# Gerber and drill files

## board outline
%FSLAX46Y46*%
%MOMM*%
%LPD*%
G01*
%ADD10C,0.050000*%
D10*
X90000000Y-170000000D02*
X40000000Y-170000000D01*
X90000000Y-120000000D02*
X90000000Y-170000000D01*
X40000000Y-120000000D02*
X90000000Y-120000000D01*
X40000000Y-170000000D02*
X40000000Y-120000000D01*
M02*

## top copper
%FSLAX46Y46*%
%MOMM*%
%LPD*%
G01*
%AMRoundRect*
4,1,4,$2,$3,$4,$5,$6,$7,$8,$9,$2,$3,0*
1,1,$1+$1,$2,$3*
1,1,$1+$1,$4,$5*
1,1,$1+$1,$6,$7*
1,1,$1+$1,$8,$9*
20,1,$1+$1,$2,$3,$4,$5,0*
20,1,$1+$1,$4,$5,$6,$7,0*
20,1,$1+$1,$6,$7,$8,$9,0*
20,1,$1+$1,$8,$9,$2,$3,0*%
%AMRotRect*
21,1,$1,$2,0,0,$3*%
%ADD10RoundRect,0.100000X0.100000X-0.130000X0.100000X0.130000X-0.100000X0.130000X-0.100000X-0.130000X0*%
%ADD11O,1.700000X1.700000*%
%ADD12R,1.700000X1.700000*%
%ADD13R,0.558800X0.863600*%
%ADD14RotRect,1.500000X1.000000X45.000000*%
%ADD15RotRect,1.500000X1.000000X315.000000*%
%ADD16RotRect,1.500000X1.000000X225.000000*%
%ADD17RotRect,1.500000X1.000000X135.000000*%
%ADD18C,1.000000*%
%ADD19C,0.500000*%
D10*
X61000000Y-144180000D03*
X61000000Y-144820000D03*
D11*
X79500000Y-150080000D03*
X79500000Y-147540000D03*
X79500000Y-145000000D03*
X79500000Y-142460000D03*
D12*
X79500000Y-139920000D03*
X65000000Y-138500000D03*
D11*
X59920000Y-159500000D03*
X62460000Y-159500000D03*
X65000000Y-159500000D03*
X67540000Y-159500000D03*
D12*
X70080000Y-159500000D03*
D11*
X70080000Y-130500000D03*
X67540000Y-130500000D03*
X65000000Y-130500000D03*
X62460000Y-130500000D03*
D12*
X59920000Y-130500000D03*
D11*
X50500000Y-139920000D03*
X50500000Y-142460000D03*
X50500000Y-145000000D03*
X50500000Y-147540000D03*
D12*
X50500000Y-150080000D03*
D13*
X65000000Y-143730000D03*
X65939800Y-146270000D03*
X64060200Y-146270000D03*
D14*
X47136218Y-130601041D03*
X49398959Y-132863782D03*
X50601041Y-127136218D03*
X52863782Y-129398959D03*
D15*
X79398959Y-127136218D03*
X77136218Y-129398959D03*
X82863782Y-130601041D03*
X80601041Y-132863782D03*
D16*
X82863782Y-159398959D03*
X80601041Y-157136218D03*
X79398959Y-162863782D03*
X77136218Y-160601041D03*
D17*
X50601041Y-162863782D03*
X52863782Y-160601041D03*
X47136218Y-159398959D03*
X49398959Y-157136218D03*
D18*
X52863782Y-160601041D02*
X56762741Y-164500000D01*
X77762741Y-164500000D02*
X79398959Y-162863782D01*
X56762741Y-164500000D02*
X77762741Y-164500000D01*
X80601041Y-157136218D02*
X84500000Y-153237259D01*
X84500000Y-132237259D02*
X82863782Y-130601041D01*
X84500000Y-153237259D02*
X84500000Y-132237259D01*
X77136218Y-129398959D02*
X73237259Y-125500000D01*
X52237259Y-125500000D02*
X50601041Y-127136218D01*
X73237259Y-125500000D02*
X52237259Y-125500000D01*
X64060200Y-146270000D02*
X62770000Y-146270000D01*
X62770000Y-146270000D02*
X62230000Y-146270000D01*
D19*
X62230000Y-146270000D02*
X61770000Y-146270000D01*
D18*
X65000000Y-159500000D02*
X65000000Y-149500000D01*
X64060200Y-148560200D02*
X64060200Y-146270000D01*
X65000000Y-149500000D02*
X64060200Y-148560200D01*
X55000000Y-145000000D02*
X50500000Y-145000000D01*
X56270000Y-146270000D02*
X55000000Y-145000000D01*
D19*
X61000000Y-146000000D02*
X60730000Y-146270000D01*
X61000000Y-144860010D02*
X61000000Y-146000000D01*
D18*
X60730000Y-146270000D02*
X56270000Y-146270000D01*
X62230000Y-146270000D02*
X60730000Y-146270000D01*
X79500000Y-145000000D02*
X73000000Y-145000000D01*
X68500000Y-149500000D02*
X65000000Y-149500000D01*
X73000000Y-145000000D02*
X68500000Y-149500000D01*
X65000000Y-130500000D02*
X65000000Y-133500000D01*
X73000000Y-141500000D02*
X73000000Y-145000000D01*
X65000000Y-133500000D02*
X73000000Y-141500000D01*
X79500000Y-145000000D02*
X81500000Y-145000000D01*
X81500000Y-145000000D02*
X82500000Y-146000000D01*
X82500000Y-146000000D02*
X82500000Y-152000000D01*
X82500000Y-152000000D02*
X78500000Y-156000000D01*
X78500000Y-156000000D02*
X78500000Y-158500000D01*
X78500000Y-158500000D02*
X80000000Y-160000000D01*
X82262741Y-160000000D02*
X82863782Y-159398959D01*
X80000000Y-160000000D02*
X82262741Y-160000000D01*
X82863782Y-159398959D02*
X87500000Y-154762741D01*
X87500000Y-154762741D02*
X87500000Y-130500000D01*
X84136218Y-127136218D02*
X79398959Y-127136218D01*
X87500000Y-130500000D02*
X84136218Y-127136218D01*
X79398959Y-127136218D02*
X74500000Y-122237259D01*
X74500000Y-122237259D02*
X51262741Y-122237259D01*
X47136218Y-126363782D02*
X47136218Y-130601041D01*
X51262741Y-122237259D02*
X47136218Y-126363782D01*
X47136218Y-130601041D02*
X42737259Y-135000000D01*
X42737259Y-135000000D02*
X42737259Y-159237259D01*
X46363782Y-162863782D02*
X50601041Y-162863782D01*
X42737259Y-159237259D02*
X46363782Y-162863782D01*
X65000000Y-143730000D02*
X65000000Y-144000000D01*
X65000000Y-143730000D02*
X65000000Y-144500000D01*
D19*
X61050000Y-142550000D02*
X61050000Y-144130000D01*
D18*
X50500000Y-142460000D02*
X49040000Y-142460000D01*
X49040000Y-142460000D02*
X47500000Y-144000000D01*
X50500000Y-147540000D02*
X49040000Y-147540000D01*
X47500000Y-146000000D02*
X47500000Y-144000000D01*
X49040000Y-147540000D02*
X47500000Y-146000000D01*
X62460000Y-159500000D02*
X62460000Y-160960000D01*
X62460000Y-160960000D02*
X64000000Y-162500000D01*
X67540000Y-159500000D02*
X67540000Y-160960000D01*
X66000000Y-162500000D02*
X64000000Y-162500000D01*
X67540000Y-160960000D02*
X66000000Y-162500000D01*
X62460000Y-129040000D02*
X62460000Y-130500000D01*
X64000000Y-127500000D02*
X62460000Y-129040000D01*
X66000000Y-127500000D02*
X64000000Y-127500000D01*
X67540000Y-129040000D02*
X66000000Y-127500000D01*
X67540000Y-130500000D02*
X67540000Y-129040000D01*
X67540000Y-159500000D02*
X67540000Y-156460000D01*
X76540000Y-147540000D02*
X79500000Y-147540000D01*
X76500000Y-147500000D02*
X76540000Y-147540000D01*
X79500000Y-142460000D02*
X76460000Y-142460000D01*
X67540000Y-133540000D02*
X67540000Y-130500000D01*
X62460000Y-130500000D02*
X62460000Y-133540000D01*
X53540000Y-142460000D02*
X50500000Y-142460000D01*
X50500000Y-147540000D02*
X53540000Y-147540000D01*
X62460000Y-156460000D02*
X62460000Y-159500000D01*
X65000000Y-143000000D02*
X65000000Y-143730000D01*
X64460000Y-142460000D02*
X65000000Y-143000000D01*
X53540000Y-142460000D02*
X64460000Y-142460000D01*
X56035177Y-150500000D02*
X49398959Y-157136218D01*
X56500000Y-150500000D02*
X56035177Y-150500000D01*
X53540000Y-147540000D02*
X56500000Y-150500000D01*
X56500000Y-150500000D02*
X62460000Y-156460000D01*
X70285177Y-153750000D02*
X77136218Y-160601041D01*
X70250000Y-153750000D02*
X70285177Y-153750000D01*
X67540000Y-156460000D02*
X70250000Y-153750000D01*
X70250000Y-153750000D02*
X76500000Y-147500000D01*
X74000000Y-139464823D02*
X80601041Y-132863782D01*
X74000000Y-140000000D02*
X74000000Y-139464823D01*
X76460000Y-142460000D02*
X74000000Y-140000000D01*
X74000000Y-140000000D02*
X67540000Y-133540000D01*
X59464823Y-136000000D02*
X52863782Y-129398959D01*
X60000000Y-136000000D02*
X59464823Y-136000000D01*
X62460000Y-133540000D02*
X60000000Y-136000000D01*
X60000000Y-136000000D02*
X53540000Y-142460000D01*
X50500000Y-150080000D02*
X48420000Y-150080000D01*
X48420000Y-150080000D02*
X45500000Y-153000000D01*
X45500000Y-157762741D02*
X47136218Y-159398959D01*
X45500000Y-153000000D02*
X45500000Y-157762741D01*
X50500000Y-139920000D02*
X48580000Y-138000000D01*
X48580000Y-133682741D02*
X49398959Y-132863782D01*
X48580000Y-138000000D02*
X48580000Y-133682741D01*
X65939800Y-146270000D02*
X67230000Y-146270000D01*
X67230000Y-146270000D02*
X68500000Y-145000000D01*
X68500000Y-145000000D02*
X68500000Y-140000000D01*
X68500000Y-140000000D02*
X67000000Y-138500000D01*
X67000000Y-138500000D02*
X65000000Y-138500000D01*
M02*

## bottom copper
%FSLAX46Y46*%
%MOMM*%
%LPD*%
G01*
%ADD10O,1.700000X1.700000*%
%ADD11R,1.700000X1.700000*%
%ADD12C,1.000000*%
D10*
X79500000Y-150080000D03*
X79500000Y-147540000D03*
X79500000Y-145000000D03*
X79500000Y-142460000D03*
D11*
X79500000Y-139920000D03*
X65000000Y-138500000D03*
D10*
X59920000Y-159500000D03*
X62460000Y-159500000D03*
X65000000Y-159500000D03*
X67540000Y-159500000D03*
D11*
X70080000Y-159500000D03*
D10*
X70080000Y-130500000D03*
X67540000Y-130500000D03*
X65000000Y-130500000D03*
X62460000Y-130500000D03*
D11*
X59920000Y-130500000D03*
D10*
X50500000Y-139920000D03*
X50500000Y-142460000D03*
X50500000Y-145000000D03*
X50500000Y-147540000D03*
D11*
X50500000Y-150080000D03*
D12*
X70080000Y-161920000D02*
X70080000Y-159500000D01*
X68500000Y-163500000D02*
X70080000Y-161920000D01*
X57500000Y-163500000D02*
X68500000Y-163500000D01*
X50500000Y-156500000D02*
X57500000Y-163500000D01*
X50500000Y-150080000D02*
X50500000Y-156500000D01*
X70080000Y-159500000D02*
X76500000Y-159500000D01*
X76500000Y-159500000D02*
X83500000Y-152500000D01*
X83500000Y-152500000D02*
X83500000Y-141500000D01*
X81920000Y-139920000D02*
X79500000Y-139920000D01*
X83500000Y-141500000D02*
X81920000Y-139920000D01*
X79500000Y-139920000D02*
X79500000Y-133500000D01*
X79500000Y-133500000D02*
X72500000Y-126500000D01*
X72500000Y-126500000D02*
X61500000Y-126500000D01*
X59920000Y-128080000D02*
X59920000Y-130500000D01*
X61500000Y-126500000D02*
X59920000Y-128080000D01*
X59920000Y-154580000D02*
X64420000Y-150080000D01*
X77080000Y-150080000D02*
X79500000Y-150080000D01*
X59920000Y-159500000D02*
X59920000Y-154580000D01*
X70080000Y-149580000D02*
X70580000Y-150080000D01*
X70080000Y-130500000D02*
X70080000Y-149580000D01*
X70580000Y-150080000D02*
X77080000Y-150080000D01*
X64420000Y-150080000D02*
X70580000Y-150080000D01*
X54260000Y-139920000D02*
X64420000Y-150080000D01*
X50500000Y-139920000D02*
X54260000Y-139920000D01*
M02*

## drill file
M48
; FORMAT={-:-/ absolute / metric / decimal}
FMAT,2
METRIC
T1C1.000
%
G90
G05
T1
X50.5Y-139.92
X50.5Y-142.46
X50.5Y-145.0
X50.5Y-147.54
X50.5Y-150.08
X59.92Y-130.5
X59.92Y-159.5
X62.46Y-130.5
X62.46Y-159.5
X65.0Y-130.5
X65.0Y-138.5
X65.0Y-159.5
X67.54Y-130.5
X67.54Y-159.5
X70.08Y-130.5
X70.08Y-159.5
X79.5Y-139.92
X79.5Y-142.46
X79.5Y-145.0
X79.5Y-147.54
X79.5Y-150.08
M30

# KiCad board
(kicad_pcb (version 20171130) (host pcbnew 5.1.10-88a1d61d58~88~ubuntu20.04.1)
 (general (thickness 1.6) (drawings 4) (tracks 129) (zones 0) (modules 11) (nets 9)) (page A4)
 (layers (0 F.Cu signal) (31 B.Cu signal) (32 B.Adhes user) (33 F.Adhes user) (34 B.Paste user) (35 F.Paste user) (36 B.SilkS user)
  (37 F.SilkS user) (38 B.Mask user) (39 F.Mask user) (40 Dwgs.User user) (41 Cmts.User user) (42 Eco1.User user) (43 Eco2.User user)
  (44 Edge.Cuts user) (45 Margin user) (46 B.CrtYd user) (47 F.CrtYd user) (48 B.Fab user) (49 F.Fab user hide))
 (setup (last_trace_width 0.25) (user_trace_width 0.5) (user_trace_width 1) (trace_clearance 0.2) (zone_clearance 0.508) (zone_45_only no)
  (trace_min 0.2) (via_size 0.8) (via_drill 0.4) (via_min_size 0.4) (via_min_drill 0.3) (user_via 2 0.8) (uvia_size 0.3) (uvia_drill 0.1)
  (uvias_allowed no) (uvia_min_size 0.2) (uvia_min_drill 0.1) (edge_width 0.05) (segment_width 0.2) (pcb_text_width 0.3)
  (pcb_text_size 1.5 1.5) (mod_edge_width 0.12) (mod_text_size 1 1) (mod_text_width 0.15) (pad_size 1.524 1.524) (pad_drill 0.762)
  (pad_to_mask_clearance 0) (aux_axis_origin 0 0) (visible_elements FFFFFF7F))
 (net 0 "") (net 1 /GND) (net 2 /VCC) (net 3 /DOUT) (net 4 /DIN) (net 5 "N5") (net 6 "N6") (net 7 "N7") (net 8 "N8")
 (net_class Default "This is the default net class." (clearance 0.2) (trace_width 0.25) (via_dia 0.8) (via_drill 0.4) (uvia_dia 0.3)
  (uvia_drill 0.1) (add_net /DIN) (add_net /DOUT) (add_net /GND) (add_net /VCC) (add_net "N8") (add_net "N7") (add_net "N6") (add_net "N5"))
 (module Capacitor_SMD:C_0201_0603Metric (layer F.Cu) (at 61 144.5 90)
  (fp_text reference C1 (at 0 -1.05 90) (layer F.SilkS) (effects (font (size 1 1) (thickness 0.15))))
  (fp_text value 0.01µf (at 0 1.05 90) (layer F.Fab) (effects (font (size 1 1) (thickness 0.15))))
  (pad 2 smd roundrect (at 0.32 0 90) (size 0.46 0.4) (layers F.Cu F.Mask) (roundrect_rratio 0.25) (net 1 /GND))
  (pad 1 smd roundrect (at -0.32 0 90) (size 0.46 0.4) (layers F.Cu F.Mask) (roundrect_rratio 0.25) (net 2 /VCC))
  (pad "" smd roundrect (at 0.345 0 90) (size 0.318 0.36) (layers F.Paste) (roundrect_rratio 0.25))
  (pad "" smd roundrect (at -0.345 0 90) (size 0.318 0.36) (layers F.Paste) (roundrect_rratio 0.25)))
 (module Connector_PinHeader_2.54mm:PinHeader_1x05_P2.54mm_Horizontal (layer F.Cu) (at 79.5 139.92)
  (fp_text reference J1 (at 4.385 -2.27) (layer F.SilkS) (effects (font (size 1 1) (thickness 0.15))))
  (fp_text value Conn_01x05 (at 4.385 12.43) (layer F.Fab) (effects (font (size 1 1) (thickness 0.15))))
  (pad 5 thru_hole oval (at 0 10.16) (size 1.7 1.7) (drill 1) (layers *.Cu *.Mask) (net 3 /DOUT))
  (pad 4 thru_hole oval (at 0 7.62) (size 1.7 1.7) (drill 1) (layers *.Cu *.Mask) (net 1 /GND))
  (pad 3 thru_hole oval (at 0 5.08) (size 1.7 1.7) (drill 1) (layers *.Cu *.Mask) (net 2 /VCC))
  (pad 2 thru_hole oval (at 0 2.54) (size 1.7 1.7) (drill 1) (layers *.Cu *.Mask) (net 1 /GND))
  (pad 1 thru_hole rect (at 0 0) (size 1.7 1.7) (drill 1) (layers *.Cu *.Mask) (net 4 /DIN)))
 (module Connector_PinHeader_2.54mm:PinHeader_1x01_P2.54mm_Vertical (layer F.Cu) (at 65 138.5)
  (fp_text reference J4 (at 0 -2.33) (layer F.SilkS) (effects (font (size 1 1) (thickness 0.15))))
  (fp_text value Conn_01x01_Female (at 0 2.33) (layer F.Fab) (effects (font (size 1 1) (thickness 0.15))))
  (pad 1 thru_hole rect (at 0 0) (size 1.7 1.7) (drill 1) (layers *.Cu *.Mask) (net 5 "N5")))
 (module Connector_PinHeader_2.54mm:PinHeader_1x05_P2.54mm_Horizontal (layer F.Cu) (at 70.08 159.5 270)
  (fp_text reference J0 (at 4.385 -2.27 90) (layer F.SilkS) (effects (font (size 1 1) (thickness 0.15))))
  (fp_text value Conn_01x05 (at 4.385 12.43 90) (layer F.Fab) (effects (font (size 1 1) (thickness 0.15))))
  (pad 5 thru_hole oval (at 0 10.16 270) (size 1.7 1.7) (drill 1) (layers *.Cu *.Mask) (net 3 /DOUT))
  (pad 4 thru_hole oval (at 0 7.62 270) (size 1.7 1.7) (drill 1) (layers *.Cu *.Mask) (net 1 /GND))
  (pad 3 thru_hole oval (at 0 5.08 270) (size 1.7 1.7) (drill 1) (layers *.Cu *.Mask) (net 2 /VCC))
  (pad 2 thru_hole oval (at 0 2.54 270) (size 1.7 1.7) (drill 1) (layers *.Cu *.Mask) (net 1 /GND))
  (pad 1 thru_hole rect (at 0 0 270) (size 1.7 1.7) (drill 1) (layers *.Cu *.Mask) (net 4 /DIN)))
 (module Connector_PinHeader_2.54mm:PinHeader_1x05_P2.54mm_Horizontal (layer F.Cu) (at 59.92 130.5 90)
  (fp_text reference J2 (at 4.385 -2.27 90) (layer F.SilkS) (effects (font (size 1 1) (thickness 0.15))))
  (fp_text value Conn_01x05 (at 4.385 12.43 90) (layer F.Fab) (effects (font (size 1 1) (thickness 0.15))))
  (pad 5 thru_hole oval (at 0 10.16 90) (size 1.7 1.7) (drill 1) (layers *.Cu *.Mask) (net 3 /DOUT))
  (pad 4 thru_hole oval (at 0 7.62 90) (size 1.7 1.7) (drill 1) (layers *.Cu *.Mask) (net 1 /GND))
  (pad 3 thru_hole oval (at 0 5.08 90) (size 1.7 1.7) (drill 1) (layers *.Cu *.Mask) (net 2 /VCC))
  (pad 2 thru_hole oval (at 0 2.54 90) (size 1.7 1.7) (drill 1) (layers *.Cu *.Mask) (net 1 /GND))
  (pad 1 thru_hole rect (at 0 0 90) (size 1.7 1.7) (drill 1) (layers *.Cu *.Mask) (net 4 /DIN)))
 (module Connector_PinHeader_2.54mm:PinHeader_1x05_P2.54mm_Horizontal (layer F.Cu) (at 50.5 150.08 180)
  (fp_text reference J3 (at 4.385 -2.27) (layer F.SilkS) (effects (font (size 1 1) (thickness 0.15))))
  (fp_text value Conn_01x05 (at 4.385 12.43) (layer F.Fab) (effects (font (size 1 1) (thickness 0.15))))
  (pad 5 thru_hole oval (at 0 10.16 180) (size 1.7 1.7) (drill 1) (layers *.Cu *.Mask) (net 3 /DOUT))
  (pad 4 thru_hole oval (at 0 7.62 180) (size 1.7 1.7) (drill 1) (layers *.Cu *.Mask) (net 1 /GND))
  (pad 3 thru_hole oval (at 0 5.08 180) (size 1.7 1.7) (drill 1) (layers *.Cu *.Mask) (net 2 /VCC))
  (pad 2 thru_hole oval (at 0 2.54 180) (size 1.7 1.7) (drill 1) (layers *.Cu *.Mask) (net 1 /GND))
  (pad 1 thru_hole rect (at 0 0 180) (size 1.7 1.7) (drill 1) (layers *.Cu *.Mask) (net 4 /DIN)))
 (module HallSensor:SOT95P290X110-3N (layer F.Cu) (at 65 145 90)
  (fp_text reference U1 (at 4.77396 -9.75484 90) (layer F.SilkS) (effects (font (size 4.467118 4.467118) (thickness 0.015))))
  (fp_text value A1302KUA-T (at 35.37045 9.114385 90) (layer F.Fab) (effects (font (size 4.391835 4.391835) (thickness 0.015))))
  (pad 3 smd rect (at 1.27 0 90) (size 0.8636 0.5588) (layers F.Cu F.Paste F.Mask) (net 1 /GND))
  (pad 2 smd rect (at -1.27 0.9398 90) (size 0.8636 0.5588) (layers F.Cu F.Paste F.Mask) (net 5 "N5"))
  (pad 1 smd rect (at -1.27 -0.9398 90) (size 0.8636 0.5588) (layers F.Cu F.Paste F.Mask) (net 2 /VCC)))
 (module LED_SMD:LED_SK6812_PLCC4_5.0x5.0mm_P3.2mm (layer F.Cu) (at 50 130 45)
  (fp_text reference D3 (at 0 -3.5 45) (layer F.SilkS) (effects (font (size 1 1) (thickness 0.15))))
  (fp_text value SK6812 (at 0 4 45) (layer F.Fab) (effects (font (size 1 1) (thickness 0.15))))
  (pad 3 smd rect (at -2.45 -1.6 45) (size 1.5 1) (layers F.Cu F.Paste F.Mask) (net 2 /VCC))
  (pad 4 smd rect (at -2.45 1.6 45) (size 1.5 1) (layers F.Cu F.Paste F.Mask) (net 3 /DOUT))
  (pad 2 smd rect (at 2.45 -1.6 45) (size 1.5 1) (layers F.Cu F.Paste F.Mask) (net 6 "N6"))
  (pad 1 smd rect (at 2.45 1.6 45) (size 1.5 1) (layers F.Cu F.Paste F.Mask) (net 1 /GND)))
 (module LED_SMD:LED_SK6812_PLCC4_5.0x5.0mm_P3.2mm (layer F.Cu) (at 80 130 315)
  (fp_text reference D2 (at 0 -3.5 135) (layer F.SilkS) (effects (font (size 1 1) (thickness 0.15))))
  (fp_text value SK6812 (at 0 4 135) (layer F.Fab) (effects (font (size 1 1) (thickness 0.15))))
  (pad 3 smd rect (at -2.45 -1.6 315) (size 1.5 1) (layers F.Cu F.Paste F.Mask) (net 2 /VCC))
  (pad 4 smd rect (at -2.45 1.6 315) (size 1.5 1) (layers F.Cu F.Paste F.Mask) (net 6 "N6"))
  (pad 2 smd rect (at 2.45 -1.6 315) (size 1.5 1) (layers F.Cu F.Paste F.Mask) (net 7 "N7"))
  (pad 1 smd rect (at 2.45 1.6 315) (size 1.5 1) (layers F.Cu F.Paste F.Mask) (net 1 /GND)))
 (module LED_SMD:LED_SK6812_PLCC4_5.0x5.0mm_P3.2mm (layer F.Cu) (at 80 160 225)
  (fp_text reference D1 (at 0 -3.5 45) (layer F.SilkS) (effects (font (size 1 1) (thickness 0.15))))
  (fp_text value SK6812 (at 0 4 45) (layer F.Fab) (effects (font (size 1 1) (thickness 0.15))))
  (pad 3 smd rect (at -2.45 -1.6 225) (size 1.5 1) (layers F.Cu F.Paste F.Mask) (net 2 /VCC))
  (pad 4 smd rect (at -2.45 1.6 225) (size 1.5 1) (layers F.Cu F.Paste F.Mask) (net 7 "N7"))
  (pad 2 smd rect (at 2.45 -1.6 225) (size 1.5 1) (layers F.Cu F.Paste F.Mask) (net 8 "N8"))
  (pad 1 smd rect (at 2.45 1.6 225) (size 1.5 1) (layers F.Cu F.Paste F.Mask) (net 1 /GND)))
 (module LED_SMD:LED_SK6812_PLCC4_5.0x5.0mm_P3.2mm (layer F.Cu) (at 50 160 135)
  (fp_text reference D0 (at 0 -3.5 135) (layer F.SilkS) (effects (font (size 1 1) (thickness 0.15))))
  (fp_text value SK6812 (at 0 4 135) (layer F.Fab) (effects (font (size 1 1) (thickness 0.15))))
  (pad 3 smd rect (at -2.45 -1.6 135) (size 1.5 1) (layers F.Cu F.Paste F.Mask) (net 2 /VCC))
  (pad 4 smd rect (at -2.45 1.6 135) (size 1.5 1) (layers F.Cu F.Paste F.Mask) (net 8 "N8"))
  (pad 2 smd rect (at 2.45 -1.6 135) (size 1.5 1) (layers F.Cu F.Paste F.Mask) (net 4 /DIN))
  (pad 1 smd rect (at 2.45 1.6 135) (size 1.5 1) (layers F.Cu F.Paste F.Mask) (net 1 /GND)))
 (gr_line (start 90 170) (end 40 170) (layer Edge.Cuts) (width 0.05))
 (gr_line (start 90 120) (end 90 170) (layer Edge.Cuts) (width 0.05))
 (gr_line (start 40 120) (end 90 120) (layer Edge.Cuts) (width 0.05))
 (gr_line (start 40 170) (end 40 120) (layer Edge.Cuts) (width 0.05))
 (segment (start 52.863782 160.601041) (end 56.762741 164.5) (width 1) (layer F.Cu) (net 8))
 (segment (start 77.762741 164.5) (end 79.398959 162.863782) (width 1) (layer F.Cu) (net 8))
 (segment (start 56.762741 164.5) (end 77.762741 164.5) (width 1) (layer F.Cu) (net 8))
 (segment (start 80.601041 157.136218) (end 84.5 153.237259) (width 1) (layer F.Cu) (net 7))
 (segment (start 84.5 132.237259) (end 82.863782 130.601041) (width 1) (layer F.Cu) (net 7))
 (segment (start 84.5 153.237259) (end 84.5 132.237259) (width 1) (layer F.Cu) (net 7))
 (segment (start 77.136218 129.398959) (end 73.237259 125.5) (width 1) (layer F.Cu) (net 6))
 (segment (start 52.237259 125.5) (end 50.601041 127.136218) (width 1) (layer F.Cu) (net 6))
 (segment (start 73.237259 125.5) (end 52.237259 125.5) (width 1) (layer F.Cu) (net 6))
 (segment (start 64.0602 146.27) (end 62.77 146.27) (width 1) (layer F.Cu) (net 2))
 (segment (start 62.77 146.27) (end 62.23 146.27) (width 1) (layer F.Cu) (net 2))
 (segment (start 62.23 146.27) (end 61.77 146.27) (width 0.5) (layer F.Cu) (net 2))
 (segment (start 65 159.5) (end 65 149.5) (width 1) (layer F.Cu) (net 2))
 (segment (start 64.0602 148.5602) (end 64.0602 146.27) (width 1) (layer F.Cu) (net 2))
 (segment (start 65 149.5) (end 64.0602 148.5602) (width 1) (layer F.Cu) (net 2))
 (segment (start 55 145) (end 50.5 145) (width 1) (layer F.Cu) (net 2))
 (segment (start 56.27 146.27) (end 55 145) (width 1) (layer F.Cu) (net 2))
 (segment (start 61 146) (end 60.73 146.27) (width 0.5) (layer F.Cu) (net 2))
 (segment (start 61 144.86001) (end 61 146) (width 0.5) (layer F.Cu) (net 2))
 (segment (start 60.73 146.27) (end 56.27 146.27) (width 1) (layer F.Cu) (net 2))
 (segment (start 62.23 146.27) (end 60.73 146.27) (width 1) (layer F.Cu) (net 2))
 (segment (start 79.5 145) (end 73 145) (width 1) (layer F.Cu) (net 2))
 (segment (start 68.5 149.5) (end 65 149.5) (width 1) (layer F.Cu) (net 2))
 (segment (start 73 145) (end 68.5 149.5) (width 1) (layer F.Cu) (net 2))
 (segment (start 65 130.5) (end 65 133.5) (width 1) (layer F.Cu) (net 2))
 (segment (start 73 141.5) (end 73 145) (width 1) (layer F.Cu) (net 2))
 (segment (start 65 133.5) (end 73 141.5) (width 1) (layer F.Cu) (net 2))
 (segment (start 79.5 145) (end 81.5 145) (width 1) (layer F.Cu) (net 2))
 (segment (start 81.5 145) (end 82.5 146) (width 1) (layer F.Cu) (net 2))
 (segment (start 82.5 146) (end 82.5 152) (width 1) (layer F.Cu) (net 2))
 (segment (start 82.5 152) (end 78.5 156) (width 1) (layer F.Cu) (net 2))
 (segment (start 78.5 156) (end 78.5 158.5) (width 1) (layer F.Cu) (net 2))
 (segment (start 78.5 158.5) (end 80 160) (width 1) (layer F.Cu) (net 2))
 (segment (start 82.262741 160) (end 82.863782 159.398959) (width 1) (layer F.Cu) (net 2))
 (segment (start 80 160) (end 82.262741 160) (width 1) (layer F.Cu) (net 2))
 (segment (start 82.863782 159.398959) (end 87.5 154.762741) (width 1) (layer F.Cu) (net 2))
 (segment (start 87.5 154.762741) (end 87.5 130.5) (width 1) (layer F.Cu) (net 2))
 (segment (start 84.136218 127.136218) (end 79.398959 127.136218) (width 1) (layer F.Cu) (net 2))
 (segment (start 87.5 130.5) (end 84.136218 127.136218) (width 1) (layer F.Cu) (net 2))
 (segment (start 79.398959 127.136218) (end 74.5 122.237259) (width 1) (layer F.Cu) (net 2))
 (segment (start 74.5 122.237259) (end 51.262741 122.237259) (width 1) (layer F.Cu) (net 2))
 (segment (start 47.136218 126.363782) (end 47.136218 130.601041) (width 1) (layer F.Cu) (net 2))
 (segment (start 51.262741 122.237259) (end 47.136218 126.363782) (width 1) (layer F.Cu) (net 2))
 (segment (start 47.136218 130.601041) (end 42.737259 135) (width 1) (layer F.Cu) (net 2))
 (segment (start 42.737259 135) (end 42.737259 159.237259) (width 1) (layer F.Cu) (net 2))
 (segment (start 46.363782 162.863782) (end 50.601041 162.863782) (width 1) (layer F.Cu) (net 2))
 (segment (start 42.737259 159.237259) (end 46.363782 162.863782) (width 1) (layer F.Cu) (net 2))
 (segment (start 65 143.73) (end 65 144) (width 1) (layer F.Cu) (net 1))
 (segment (start 65 143.73) (end 65 144.5) (width 1) (layer F.Cu) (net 1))
 (segment (start 61.05 142.55) (end 61.05 144.13) (width 0.5) (layer F.Cu) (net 1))
 (segment (start 50.5 142.46) (end 49.04 142.46) (width 1) (layer F.Cu) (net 1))
 (segment (start 49.04 142.46) (end 47.5 144) (width 1) (layer F.Cu) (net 1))
 (segment (start 50.5 147.54) (end 49.04 147.54) (width 1) (layer F.Cu) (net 1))
 (segment (start 47.5 146) (end 47.5 144) (width 1) (layer F.Cu) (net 1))
 (segment (start 49.04 147.54) (end 47.5 146) (width 1) (layer F.Cu) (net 1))
 (segment (start 62.46 159.5) (end 62.46 160.96) (width 1) (layer F.Cu) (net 1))
 (segment (start 62.46 160.96) (end 64 162.5) (width 1) (layer F.Cu) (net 1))
 (segment (start 67.54 159.5) (end 67.54 160.96) (width 1) (layer F.Cu) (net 1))
 (segment (start 66 162.5) (end 64 162.5) (width 1) (layer F.Cu) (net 1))
 (segment (start 67.54 160.96) (end 66 162.5) (width 1) (layer F.Cu) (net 1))
 (segment (start 62.46 129.04) (end 62.46 130.5) (width 1) (layer F.Cu) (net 1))
 (segment (start 64 127.5) (end 62.46 129.04) (width 1) (layer F.Cu) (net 1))
 (segment (start 66 127.5) (end 64 127.5) (width 1) (layer F.Cu) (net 1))
 (segment (start 67.54 129.04) (end 66 127.5) (width 1) (layer F.Cu) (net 1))
 (segment (start 67.54 130.5) (end 67.54 129.04) (width 1) (layer F.Cu) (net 1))
 (segment (start 67.54 159.5) (end 67.54 156.46) (width 1) (layer F.Cu) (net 1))
 (segment (start 76.54 147.54) (end 79.5 147.54) (width 1) (layer F.Cu) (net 1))
 (segment (start 76.5 147.5) (end 76.54 147.54) (width 1) (layer F.Cu) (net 1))
 (segment (start 79.5 142.46) (end 76.46 142.46) (width 1) (layer F.Cu) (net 1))
 (segment (start 67.54 133.54) (end 67.54 130.5) (width 1) (layer F.Cu) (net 1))
 (segment (start 62.46 130.5) (end 62.46 133.54) (width 1) (layer F.Cu) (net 1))
 (segment (start 53.54 142.46) (end 50.5 142.46) (width 1) (layer F.Cu) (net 1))
 (segment (start 50.5 147.54) (end 53.54 147.54) (width 1) (layer F.Cu) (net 1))
 (segment (start 62.46 156.46) (end 62.46 159.5) (width 1) (layer F.Cu) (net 1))
 (segment (start 65 143) (end 65 143.73) (width 1) (layer F.Cu) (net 1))
 (segment (start 64.46 142.46) (end 65 143) (width 1) (layer F.Cu) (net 1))
 (segment (start 53.54 142.46) (end 64.46 142.46) (width 1) (layer F.Cu) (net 1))
 (segment (start 56.035177 150.5) (end 49.398959 157.136218) (width 1) (layer F.Cu) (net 1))
 (segment (start 56.5 150.5) (end 56.035177 150.5) (width 1) (layer F.Cu) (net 1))
 (segment (start 53.54 147.54) (end 56.5 150.5) (width 1) (layer F.Cu) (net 1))
 (segment (start 56.5 150.5) (end 62.46 156.46) (width 1) (layer F.Cu) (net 1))
 (segment (start 70.285177 153.75) (end 77.136218 160.601041) (width 1) (layer F.Cu) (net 1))
 (segment (start 70.25 153.75) (end 70.285177 153.75) (width 1) (layer F.Cu) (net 1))
 (segment (start 67.54 156.46) (end 70.25 153.75) (width 1) (layer F.Cu) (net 1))
 (segment (start 70.25 153.75) (end 76.5 147.5) (width 1) (layer F.Cu) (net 1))
 (segment (start 74 139.464823) (end 80.601041 132.863782) (width 1) (layer F.Cu) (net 1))
 (segment (start 74 140) (end 74 139.464823) (width 1) (layer F.Cu) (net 1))
 (segment (start 76.46 142.46) (end 74 140) (width 1) (layer F.Cu) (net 1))
 (segment (start 74 140) (end 67.54 133.54) (width 1) (layer F.Cu) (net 1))
 (segment (start 59.464823 136) (end 52.863782 129.398959) (width 1) (layer F.Cu) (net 1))
 (segment (start 60 136) (end 59.464823 136) (width 1) (layer F.Cu) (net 1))
 (segment (start 62.46 133.54) (end 60 136) (width 1) (layer F.Cu) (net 1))
 (segment (start 60 136) (end 53.54 142.46) (width 1) (layer F.Cu) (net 1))
 (segment (start 50.5 150.08) (end 48.42 150.08) (width 1) (layer F.Cu) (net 4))
 (segment (start 48.42 150.08) (end 45.5 153) (width 1) (layer F.Cu) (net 4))
 (segment (start 45.5 157.762741) (end 47.136218 159.398959) (width 1) (layer F.Cu) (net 4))
 (segment (start 45.5 153) (end 45.5 157.762741) (width 1) (layer F.Cu) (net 4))
 (segment (start 70.08 161.92) (end 70.08 159.5) (width 1) (layer B.Cu) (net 4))
 (segment (start 68.5 163.5) (end 70.08 161.92) (width 1) (layer B.Cu) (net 4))
 (segment (start 57.5 163.5) (end 68.5 163.5) (width 1) (layer B.Cu) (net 4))
 (segment (start 50.5 156.5) (end 57.5 163.5) (width 1) (layer B.Cu) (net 4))
 (segment (start 50.5 150.08) (end 50.5 156.5) (width 1) (layer B.Cu) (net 4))
 (segment (start 70.08 159.5) (end 76.5 159.5) (width 1) (layer B.Cu) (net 4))
 (segment (start 76.5 159.5) (end 83.5 152.5) (width 1) (layer B.Cu) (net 4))
 (segment (start 83.5 152.5) (end 83.5 141.5) (width 1) (layer B.Cu) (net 4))
 (segment (start 81.92 139.92) (end 79.5 139.92) (width 1) (layer B.Cu) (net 4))
 (segment (start 83.5 141.5) (end 81.92 139.92) (width 1) (layer B.Cu) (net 4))
 (segment (start 79.5 139.92) (end 79.5 133.5) (width 1) (layer B.Cu) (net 4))
 (segment (start 79.5 133.5) (end 72.5 126.5) (width 1) (layer B.Cu) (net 4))
 (segment (start 72.5 126.5) (end 61.5 126.5) (width 1) (layer B.Cu) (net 4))
 (segment (start 59.92 128.08) (end 59.92 130.5) (width 1) (layer B.Cu) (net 4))
 (segment (start 61.5 126.5) (end 59.92 128.08) (width 1) (layer B.Cu) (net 4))
 (segment (start 50.5 139.92) (end 48.58 138) (width 1) (layer F.Cu) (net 3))
 (segment (start 48.58 133.682741) (end 49.398959 132.863782) (width 1) (layer F.Cu) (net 3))
 (segment (start 48.58 138) (end 48.58 133.682741) (width 1) (layer F.Cu) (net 3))
 (segment (start 59.92 154.58) (end 64.42 150.08) (width 1) (layer B.Cu) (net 3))
 (segment (start 77.08 150.08) (end 79.5 150.08) (width 1) (layer B.Cu) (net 3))
 (segment (start 59.92 159.5) (end 59.92 154.58) (width 1) (layer B.Cu) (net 3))
 (segment (start 70.08 149.58) (end 70.58 150.08) (width 1) (layer B.Cu) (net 3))
 (segment (start 70.08 130.5) (end 70.08 149.58) (width 1) (layer B.Cu) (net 3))
 (segment (start 70.58 150.08) (end 77.08 150.08) (width 1) (layer B.Cu) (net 3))
 (segment (start 64.42 150.08) (end 70.58 150.08) (width 1) (layer B.Cu) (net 3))
 (segment (start 54.26 139.92) (end 64.42 150.08) (width 1) (layer B.Cu) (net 3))
 (segment (start 50.5 139.92) (end 54.26 139.92) (width 1) (layer B.Cu) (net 3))
 (segment (start 65.9398 146.27) (end 67.23 146.27) (width 1) (layer F.Cu) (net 5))
 (segment (start 67.23 146.27) (end 68.5 145) (width 1) (layer F.Cu) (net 5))
 (segment (start 68.5 145) (end 68.5 140) (width 1) (layer F.Cu) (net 5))
 (segment (start 68.5 140) (end 67 138.5) (width 1) (layer F.Cu) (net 5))
 (segment (start 67 138.5) (end 65 138.5) (width 1) (layer F.Cu) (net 5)))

